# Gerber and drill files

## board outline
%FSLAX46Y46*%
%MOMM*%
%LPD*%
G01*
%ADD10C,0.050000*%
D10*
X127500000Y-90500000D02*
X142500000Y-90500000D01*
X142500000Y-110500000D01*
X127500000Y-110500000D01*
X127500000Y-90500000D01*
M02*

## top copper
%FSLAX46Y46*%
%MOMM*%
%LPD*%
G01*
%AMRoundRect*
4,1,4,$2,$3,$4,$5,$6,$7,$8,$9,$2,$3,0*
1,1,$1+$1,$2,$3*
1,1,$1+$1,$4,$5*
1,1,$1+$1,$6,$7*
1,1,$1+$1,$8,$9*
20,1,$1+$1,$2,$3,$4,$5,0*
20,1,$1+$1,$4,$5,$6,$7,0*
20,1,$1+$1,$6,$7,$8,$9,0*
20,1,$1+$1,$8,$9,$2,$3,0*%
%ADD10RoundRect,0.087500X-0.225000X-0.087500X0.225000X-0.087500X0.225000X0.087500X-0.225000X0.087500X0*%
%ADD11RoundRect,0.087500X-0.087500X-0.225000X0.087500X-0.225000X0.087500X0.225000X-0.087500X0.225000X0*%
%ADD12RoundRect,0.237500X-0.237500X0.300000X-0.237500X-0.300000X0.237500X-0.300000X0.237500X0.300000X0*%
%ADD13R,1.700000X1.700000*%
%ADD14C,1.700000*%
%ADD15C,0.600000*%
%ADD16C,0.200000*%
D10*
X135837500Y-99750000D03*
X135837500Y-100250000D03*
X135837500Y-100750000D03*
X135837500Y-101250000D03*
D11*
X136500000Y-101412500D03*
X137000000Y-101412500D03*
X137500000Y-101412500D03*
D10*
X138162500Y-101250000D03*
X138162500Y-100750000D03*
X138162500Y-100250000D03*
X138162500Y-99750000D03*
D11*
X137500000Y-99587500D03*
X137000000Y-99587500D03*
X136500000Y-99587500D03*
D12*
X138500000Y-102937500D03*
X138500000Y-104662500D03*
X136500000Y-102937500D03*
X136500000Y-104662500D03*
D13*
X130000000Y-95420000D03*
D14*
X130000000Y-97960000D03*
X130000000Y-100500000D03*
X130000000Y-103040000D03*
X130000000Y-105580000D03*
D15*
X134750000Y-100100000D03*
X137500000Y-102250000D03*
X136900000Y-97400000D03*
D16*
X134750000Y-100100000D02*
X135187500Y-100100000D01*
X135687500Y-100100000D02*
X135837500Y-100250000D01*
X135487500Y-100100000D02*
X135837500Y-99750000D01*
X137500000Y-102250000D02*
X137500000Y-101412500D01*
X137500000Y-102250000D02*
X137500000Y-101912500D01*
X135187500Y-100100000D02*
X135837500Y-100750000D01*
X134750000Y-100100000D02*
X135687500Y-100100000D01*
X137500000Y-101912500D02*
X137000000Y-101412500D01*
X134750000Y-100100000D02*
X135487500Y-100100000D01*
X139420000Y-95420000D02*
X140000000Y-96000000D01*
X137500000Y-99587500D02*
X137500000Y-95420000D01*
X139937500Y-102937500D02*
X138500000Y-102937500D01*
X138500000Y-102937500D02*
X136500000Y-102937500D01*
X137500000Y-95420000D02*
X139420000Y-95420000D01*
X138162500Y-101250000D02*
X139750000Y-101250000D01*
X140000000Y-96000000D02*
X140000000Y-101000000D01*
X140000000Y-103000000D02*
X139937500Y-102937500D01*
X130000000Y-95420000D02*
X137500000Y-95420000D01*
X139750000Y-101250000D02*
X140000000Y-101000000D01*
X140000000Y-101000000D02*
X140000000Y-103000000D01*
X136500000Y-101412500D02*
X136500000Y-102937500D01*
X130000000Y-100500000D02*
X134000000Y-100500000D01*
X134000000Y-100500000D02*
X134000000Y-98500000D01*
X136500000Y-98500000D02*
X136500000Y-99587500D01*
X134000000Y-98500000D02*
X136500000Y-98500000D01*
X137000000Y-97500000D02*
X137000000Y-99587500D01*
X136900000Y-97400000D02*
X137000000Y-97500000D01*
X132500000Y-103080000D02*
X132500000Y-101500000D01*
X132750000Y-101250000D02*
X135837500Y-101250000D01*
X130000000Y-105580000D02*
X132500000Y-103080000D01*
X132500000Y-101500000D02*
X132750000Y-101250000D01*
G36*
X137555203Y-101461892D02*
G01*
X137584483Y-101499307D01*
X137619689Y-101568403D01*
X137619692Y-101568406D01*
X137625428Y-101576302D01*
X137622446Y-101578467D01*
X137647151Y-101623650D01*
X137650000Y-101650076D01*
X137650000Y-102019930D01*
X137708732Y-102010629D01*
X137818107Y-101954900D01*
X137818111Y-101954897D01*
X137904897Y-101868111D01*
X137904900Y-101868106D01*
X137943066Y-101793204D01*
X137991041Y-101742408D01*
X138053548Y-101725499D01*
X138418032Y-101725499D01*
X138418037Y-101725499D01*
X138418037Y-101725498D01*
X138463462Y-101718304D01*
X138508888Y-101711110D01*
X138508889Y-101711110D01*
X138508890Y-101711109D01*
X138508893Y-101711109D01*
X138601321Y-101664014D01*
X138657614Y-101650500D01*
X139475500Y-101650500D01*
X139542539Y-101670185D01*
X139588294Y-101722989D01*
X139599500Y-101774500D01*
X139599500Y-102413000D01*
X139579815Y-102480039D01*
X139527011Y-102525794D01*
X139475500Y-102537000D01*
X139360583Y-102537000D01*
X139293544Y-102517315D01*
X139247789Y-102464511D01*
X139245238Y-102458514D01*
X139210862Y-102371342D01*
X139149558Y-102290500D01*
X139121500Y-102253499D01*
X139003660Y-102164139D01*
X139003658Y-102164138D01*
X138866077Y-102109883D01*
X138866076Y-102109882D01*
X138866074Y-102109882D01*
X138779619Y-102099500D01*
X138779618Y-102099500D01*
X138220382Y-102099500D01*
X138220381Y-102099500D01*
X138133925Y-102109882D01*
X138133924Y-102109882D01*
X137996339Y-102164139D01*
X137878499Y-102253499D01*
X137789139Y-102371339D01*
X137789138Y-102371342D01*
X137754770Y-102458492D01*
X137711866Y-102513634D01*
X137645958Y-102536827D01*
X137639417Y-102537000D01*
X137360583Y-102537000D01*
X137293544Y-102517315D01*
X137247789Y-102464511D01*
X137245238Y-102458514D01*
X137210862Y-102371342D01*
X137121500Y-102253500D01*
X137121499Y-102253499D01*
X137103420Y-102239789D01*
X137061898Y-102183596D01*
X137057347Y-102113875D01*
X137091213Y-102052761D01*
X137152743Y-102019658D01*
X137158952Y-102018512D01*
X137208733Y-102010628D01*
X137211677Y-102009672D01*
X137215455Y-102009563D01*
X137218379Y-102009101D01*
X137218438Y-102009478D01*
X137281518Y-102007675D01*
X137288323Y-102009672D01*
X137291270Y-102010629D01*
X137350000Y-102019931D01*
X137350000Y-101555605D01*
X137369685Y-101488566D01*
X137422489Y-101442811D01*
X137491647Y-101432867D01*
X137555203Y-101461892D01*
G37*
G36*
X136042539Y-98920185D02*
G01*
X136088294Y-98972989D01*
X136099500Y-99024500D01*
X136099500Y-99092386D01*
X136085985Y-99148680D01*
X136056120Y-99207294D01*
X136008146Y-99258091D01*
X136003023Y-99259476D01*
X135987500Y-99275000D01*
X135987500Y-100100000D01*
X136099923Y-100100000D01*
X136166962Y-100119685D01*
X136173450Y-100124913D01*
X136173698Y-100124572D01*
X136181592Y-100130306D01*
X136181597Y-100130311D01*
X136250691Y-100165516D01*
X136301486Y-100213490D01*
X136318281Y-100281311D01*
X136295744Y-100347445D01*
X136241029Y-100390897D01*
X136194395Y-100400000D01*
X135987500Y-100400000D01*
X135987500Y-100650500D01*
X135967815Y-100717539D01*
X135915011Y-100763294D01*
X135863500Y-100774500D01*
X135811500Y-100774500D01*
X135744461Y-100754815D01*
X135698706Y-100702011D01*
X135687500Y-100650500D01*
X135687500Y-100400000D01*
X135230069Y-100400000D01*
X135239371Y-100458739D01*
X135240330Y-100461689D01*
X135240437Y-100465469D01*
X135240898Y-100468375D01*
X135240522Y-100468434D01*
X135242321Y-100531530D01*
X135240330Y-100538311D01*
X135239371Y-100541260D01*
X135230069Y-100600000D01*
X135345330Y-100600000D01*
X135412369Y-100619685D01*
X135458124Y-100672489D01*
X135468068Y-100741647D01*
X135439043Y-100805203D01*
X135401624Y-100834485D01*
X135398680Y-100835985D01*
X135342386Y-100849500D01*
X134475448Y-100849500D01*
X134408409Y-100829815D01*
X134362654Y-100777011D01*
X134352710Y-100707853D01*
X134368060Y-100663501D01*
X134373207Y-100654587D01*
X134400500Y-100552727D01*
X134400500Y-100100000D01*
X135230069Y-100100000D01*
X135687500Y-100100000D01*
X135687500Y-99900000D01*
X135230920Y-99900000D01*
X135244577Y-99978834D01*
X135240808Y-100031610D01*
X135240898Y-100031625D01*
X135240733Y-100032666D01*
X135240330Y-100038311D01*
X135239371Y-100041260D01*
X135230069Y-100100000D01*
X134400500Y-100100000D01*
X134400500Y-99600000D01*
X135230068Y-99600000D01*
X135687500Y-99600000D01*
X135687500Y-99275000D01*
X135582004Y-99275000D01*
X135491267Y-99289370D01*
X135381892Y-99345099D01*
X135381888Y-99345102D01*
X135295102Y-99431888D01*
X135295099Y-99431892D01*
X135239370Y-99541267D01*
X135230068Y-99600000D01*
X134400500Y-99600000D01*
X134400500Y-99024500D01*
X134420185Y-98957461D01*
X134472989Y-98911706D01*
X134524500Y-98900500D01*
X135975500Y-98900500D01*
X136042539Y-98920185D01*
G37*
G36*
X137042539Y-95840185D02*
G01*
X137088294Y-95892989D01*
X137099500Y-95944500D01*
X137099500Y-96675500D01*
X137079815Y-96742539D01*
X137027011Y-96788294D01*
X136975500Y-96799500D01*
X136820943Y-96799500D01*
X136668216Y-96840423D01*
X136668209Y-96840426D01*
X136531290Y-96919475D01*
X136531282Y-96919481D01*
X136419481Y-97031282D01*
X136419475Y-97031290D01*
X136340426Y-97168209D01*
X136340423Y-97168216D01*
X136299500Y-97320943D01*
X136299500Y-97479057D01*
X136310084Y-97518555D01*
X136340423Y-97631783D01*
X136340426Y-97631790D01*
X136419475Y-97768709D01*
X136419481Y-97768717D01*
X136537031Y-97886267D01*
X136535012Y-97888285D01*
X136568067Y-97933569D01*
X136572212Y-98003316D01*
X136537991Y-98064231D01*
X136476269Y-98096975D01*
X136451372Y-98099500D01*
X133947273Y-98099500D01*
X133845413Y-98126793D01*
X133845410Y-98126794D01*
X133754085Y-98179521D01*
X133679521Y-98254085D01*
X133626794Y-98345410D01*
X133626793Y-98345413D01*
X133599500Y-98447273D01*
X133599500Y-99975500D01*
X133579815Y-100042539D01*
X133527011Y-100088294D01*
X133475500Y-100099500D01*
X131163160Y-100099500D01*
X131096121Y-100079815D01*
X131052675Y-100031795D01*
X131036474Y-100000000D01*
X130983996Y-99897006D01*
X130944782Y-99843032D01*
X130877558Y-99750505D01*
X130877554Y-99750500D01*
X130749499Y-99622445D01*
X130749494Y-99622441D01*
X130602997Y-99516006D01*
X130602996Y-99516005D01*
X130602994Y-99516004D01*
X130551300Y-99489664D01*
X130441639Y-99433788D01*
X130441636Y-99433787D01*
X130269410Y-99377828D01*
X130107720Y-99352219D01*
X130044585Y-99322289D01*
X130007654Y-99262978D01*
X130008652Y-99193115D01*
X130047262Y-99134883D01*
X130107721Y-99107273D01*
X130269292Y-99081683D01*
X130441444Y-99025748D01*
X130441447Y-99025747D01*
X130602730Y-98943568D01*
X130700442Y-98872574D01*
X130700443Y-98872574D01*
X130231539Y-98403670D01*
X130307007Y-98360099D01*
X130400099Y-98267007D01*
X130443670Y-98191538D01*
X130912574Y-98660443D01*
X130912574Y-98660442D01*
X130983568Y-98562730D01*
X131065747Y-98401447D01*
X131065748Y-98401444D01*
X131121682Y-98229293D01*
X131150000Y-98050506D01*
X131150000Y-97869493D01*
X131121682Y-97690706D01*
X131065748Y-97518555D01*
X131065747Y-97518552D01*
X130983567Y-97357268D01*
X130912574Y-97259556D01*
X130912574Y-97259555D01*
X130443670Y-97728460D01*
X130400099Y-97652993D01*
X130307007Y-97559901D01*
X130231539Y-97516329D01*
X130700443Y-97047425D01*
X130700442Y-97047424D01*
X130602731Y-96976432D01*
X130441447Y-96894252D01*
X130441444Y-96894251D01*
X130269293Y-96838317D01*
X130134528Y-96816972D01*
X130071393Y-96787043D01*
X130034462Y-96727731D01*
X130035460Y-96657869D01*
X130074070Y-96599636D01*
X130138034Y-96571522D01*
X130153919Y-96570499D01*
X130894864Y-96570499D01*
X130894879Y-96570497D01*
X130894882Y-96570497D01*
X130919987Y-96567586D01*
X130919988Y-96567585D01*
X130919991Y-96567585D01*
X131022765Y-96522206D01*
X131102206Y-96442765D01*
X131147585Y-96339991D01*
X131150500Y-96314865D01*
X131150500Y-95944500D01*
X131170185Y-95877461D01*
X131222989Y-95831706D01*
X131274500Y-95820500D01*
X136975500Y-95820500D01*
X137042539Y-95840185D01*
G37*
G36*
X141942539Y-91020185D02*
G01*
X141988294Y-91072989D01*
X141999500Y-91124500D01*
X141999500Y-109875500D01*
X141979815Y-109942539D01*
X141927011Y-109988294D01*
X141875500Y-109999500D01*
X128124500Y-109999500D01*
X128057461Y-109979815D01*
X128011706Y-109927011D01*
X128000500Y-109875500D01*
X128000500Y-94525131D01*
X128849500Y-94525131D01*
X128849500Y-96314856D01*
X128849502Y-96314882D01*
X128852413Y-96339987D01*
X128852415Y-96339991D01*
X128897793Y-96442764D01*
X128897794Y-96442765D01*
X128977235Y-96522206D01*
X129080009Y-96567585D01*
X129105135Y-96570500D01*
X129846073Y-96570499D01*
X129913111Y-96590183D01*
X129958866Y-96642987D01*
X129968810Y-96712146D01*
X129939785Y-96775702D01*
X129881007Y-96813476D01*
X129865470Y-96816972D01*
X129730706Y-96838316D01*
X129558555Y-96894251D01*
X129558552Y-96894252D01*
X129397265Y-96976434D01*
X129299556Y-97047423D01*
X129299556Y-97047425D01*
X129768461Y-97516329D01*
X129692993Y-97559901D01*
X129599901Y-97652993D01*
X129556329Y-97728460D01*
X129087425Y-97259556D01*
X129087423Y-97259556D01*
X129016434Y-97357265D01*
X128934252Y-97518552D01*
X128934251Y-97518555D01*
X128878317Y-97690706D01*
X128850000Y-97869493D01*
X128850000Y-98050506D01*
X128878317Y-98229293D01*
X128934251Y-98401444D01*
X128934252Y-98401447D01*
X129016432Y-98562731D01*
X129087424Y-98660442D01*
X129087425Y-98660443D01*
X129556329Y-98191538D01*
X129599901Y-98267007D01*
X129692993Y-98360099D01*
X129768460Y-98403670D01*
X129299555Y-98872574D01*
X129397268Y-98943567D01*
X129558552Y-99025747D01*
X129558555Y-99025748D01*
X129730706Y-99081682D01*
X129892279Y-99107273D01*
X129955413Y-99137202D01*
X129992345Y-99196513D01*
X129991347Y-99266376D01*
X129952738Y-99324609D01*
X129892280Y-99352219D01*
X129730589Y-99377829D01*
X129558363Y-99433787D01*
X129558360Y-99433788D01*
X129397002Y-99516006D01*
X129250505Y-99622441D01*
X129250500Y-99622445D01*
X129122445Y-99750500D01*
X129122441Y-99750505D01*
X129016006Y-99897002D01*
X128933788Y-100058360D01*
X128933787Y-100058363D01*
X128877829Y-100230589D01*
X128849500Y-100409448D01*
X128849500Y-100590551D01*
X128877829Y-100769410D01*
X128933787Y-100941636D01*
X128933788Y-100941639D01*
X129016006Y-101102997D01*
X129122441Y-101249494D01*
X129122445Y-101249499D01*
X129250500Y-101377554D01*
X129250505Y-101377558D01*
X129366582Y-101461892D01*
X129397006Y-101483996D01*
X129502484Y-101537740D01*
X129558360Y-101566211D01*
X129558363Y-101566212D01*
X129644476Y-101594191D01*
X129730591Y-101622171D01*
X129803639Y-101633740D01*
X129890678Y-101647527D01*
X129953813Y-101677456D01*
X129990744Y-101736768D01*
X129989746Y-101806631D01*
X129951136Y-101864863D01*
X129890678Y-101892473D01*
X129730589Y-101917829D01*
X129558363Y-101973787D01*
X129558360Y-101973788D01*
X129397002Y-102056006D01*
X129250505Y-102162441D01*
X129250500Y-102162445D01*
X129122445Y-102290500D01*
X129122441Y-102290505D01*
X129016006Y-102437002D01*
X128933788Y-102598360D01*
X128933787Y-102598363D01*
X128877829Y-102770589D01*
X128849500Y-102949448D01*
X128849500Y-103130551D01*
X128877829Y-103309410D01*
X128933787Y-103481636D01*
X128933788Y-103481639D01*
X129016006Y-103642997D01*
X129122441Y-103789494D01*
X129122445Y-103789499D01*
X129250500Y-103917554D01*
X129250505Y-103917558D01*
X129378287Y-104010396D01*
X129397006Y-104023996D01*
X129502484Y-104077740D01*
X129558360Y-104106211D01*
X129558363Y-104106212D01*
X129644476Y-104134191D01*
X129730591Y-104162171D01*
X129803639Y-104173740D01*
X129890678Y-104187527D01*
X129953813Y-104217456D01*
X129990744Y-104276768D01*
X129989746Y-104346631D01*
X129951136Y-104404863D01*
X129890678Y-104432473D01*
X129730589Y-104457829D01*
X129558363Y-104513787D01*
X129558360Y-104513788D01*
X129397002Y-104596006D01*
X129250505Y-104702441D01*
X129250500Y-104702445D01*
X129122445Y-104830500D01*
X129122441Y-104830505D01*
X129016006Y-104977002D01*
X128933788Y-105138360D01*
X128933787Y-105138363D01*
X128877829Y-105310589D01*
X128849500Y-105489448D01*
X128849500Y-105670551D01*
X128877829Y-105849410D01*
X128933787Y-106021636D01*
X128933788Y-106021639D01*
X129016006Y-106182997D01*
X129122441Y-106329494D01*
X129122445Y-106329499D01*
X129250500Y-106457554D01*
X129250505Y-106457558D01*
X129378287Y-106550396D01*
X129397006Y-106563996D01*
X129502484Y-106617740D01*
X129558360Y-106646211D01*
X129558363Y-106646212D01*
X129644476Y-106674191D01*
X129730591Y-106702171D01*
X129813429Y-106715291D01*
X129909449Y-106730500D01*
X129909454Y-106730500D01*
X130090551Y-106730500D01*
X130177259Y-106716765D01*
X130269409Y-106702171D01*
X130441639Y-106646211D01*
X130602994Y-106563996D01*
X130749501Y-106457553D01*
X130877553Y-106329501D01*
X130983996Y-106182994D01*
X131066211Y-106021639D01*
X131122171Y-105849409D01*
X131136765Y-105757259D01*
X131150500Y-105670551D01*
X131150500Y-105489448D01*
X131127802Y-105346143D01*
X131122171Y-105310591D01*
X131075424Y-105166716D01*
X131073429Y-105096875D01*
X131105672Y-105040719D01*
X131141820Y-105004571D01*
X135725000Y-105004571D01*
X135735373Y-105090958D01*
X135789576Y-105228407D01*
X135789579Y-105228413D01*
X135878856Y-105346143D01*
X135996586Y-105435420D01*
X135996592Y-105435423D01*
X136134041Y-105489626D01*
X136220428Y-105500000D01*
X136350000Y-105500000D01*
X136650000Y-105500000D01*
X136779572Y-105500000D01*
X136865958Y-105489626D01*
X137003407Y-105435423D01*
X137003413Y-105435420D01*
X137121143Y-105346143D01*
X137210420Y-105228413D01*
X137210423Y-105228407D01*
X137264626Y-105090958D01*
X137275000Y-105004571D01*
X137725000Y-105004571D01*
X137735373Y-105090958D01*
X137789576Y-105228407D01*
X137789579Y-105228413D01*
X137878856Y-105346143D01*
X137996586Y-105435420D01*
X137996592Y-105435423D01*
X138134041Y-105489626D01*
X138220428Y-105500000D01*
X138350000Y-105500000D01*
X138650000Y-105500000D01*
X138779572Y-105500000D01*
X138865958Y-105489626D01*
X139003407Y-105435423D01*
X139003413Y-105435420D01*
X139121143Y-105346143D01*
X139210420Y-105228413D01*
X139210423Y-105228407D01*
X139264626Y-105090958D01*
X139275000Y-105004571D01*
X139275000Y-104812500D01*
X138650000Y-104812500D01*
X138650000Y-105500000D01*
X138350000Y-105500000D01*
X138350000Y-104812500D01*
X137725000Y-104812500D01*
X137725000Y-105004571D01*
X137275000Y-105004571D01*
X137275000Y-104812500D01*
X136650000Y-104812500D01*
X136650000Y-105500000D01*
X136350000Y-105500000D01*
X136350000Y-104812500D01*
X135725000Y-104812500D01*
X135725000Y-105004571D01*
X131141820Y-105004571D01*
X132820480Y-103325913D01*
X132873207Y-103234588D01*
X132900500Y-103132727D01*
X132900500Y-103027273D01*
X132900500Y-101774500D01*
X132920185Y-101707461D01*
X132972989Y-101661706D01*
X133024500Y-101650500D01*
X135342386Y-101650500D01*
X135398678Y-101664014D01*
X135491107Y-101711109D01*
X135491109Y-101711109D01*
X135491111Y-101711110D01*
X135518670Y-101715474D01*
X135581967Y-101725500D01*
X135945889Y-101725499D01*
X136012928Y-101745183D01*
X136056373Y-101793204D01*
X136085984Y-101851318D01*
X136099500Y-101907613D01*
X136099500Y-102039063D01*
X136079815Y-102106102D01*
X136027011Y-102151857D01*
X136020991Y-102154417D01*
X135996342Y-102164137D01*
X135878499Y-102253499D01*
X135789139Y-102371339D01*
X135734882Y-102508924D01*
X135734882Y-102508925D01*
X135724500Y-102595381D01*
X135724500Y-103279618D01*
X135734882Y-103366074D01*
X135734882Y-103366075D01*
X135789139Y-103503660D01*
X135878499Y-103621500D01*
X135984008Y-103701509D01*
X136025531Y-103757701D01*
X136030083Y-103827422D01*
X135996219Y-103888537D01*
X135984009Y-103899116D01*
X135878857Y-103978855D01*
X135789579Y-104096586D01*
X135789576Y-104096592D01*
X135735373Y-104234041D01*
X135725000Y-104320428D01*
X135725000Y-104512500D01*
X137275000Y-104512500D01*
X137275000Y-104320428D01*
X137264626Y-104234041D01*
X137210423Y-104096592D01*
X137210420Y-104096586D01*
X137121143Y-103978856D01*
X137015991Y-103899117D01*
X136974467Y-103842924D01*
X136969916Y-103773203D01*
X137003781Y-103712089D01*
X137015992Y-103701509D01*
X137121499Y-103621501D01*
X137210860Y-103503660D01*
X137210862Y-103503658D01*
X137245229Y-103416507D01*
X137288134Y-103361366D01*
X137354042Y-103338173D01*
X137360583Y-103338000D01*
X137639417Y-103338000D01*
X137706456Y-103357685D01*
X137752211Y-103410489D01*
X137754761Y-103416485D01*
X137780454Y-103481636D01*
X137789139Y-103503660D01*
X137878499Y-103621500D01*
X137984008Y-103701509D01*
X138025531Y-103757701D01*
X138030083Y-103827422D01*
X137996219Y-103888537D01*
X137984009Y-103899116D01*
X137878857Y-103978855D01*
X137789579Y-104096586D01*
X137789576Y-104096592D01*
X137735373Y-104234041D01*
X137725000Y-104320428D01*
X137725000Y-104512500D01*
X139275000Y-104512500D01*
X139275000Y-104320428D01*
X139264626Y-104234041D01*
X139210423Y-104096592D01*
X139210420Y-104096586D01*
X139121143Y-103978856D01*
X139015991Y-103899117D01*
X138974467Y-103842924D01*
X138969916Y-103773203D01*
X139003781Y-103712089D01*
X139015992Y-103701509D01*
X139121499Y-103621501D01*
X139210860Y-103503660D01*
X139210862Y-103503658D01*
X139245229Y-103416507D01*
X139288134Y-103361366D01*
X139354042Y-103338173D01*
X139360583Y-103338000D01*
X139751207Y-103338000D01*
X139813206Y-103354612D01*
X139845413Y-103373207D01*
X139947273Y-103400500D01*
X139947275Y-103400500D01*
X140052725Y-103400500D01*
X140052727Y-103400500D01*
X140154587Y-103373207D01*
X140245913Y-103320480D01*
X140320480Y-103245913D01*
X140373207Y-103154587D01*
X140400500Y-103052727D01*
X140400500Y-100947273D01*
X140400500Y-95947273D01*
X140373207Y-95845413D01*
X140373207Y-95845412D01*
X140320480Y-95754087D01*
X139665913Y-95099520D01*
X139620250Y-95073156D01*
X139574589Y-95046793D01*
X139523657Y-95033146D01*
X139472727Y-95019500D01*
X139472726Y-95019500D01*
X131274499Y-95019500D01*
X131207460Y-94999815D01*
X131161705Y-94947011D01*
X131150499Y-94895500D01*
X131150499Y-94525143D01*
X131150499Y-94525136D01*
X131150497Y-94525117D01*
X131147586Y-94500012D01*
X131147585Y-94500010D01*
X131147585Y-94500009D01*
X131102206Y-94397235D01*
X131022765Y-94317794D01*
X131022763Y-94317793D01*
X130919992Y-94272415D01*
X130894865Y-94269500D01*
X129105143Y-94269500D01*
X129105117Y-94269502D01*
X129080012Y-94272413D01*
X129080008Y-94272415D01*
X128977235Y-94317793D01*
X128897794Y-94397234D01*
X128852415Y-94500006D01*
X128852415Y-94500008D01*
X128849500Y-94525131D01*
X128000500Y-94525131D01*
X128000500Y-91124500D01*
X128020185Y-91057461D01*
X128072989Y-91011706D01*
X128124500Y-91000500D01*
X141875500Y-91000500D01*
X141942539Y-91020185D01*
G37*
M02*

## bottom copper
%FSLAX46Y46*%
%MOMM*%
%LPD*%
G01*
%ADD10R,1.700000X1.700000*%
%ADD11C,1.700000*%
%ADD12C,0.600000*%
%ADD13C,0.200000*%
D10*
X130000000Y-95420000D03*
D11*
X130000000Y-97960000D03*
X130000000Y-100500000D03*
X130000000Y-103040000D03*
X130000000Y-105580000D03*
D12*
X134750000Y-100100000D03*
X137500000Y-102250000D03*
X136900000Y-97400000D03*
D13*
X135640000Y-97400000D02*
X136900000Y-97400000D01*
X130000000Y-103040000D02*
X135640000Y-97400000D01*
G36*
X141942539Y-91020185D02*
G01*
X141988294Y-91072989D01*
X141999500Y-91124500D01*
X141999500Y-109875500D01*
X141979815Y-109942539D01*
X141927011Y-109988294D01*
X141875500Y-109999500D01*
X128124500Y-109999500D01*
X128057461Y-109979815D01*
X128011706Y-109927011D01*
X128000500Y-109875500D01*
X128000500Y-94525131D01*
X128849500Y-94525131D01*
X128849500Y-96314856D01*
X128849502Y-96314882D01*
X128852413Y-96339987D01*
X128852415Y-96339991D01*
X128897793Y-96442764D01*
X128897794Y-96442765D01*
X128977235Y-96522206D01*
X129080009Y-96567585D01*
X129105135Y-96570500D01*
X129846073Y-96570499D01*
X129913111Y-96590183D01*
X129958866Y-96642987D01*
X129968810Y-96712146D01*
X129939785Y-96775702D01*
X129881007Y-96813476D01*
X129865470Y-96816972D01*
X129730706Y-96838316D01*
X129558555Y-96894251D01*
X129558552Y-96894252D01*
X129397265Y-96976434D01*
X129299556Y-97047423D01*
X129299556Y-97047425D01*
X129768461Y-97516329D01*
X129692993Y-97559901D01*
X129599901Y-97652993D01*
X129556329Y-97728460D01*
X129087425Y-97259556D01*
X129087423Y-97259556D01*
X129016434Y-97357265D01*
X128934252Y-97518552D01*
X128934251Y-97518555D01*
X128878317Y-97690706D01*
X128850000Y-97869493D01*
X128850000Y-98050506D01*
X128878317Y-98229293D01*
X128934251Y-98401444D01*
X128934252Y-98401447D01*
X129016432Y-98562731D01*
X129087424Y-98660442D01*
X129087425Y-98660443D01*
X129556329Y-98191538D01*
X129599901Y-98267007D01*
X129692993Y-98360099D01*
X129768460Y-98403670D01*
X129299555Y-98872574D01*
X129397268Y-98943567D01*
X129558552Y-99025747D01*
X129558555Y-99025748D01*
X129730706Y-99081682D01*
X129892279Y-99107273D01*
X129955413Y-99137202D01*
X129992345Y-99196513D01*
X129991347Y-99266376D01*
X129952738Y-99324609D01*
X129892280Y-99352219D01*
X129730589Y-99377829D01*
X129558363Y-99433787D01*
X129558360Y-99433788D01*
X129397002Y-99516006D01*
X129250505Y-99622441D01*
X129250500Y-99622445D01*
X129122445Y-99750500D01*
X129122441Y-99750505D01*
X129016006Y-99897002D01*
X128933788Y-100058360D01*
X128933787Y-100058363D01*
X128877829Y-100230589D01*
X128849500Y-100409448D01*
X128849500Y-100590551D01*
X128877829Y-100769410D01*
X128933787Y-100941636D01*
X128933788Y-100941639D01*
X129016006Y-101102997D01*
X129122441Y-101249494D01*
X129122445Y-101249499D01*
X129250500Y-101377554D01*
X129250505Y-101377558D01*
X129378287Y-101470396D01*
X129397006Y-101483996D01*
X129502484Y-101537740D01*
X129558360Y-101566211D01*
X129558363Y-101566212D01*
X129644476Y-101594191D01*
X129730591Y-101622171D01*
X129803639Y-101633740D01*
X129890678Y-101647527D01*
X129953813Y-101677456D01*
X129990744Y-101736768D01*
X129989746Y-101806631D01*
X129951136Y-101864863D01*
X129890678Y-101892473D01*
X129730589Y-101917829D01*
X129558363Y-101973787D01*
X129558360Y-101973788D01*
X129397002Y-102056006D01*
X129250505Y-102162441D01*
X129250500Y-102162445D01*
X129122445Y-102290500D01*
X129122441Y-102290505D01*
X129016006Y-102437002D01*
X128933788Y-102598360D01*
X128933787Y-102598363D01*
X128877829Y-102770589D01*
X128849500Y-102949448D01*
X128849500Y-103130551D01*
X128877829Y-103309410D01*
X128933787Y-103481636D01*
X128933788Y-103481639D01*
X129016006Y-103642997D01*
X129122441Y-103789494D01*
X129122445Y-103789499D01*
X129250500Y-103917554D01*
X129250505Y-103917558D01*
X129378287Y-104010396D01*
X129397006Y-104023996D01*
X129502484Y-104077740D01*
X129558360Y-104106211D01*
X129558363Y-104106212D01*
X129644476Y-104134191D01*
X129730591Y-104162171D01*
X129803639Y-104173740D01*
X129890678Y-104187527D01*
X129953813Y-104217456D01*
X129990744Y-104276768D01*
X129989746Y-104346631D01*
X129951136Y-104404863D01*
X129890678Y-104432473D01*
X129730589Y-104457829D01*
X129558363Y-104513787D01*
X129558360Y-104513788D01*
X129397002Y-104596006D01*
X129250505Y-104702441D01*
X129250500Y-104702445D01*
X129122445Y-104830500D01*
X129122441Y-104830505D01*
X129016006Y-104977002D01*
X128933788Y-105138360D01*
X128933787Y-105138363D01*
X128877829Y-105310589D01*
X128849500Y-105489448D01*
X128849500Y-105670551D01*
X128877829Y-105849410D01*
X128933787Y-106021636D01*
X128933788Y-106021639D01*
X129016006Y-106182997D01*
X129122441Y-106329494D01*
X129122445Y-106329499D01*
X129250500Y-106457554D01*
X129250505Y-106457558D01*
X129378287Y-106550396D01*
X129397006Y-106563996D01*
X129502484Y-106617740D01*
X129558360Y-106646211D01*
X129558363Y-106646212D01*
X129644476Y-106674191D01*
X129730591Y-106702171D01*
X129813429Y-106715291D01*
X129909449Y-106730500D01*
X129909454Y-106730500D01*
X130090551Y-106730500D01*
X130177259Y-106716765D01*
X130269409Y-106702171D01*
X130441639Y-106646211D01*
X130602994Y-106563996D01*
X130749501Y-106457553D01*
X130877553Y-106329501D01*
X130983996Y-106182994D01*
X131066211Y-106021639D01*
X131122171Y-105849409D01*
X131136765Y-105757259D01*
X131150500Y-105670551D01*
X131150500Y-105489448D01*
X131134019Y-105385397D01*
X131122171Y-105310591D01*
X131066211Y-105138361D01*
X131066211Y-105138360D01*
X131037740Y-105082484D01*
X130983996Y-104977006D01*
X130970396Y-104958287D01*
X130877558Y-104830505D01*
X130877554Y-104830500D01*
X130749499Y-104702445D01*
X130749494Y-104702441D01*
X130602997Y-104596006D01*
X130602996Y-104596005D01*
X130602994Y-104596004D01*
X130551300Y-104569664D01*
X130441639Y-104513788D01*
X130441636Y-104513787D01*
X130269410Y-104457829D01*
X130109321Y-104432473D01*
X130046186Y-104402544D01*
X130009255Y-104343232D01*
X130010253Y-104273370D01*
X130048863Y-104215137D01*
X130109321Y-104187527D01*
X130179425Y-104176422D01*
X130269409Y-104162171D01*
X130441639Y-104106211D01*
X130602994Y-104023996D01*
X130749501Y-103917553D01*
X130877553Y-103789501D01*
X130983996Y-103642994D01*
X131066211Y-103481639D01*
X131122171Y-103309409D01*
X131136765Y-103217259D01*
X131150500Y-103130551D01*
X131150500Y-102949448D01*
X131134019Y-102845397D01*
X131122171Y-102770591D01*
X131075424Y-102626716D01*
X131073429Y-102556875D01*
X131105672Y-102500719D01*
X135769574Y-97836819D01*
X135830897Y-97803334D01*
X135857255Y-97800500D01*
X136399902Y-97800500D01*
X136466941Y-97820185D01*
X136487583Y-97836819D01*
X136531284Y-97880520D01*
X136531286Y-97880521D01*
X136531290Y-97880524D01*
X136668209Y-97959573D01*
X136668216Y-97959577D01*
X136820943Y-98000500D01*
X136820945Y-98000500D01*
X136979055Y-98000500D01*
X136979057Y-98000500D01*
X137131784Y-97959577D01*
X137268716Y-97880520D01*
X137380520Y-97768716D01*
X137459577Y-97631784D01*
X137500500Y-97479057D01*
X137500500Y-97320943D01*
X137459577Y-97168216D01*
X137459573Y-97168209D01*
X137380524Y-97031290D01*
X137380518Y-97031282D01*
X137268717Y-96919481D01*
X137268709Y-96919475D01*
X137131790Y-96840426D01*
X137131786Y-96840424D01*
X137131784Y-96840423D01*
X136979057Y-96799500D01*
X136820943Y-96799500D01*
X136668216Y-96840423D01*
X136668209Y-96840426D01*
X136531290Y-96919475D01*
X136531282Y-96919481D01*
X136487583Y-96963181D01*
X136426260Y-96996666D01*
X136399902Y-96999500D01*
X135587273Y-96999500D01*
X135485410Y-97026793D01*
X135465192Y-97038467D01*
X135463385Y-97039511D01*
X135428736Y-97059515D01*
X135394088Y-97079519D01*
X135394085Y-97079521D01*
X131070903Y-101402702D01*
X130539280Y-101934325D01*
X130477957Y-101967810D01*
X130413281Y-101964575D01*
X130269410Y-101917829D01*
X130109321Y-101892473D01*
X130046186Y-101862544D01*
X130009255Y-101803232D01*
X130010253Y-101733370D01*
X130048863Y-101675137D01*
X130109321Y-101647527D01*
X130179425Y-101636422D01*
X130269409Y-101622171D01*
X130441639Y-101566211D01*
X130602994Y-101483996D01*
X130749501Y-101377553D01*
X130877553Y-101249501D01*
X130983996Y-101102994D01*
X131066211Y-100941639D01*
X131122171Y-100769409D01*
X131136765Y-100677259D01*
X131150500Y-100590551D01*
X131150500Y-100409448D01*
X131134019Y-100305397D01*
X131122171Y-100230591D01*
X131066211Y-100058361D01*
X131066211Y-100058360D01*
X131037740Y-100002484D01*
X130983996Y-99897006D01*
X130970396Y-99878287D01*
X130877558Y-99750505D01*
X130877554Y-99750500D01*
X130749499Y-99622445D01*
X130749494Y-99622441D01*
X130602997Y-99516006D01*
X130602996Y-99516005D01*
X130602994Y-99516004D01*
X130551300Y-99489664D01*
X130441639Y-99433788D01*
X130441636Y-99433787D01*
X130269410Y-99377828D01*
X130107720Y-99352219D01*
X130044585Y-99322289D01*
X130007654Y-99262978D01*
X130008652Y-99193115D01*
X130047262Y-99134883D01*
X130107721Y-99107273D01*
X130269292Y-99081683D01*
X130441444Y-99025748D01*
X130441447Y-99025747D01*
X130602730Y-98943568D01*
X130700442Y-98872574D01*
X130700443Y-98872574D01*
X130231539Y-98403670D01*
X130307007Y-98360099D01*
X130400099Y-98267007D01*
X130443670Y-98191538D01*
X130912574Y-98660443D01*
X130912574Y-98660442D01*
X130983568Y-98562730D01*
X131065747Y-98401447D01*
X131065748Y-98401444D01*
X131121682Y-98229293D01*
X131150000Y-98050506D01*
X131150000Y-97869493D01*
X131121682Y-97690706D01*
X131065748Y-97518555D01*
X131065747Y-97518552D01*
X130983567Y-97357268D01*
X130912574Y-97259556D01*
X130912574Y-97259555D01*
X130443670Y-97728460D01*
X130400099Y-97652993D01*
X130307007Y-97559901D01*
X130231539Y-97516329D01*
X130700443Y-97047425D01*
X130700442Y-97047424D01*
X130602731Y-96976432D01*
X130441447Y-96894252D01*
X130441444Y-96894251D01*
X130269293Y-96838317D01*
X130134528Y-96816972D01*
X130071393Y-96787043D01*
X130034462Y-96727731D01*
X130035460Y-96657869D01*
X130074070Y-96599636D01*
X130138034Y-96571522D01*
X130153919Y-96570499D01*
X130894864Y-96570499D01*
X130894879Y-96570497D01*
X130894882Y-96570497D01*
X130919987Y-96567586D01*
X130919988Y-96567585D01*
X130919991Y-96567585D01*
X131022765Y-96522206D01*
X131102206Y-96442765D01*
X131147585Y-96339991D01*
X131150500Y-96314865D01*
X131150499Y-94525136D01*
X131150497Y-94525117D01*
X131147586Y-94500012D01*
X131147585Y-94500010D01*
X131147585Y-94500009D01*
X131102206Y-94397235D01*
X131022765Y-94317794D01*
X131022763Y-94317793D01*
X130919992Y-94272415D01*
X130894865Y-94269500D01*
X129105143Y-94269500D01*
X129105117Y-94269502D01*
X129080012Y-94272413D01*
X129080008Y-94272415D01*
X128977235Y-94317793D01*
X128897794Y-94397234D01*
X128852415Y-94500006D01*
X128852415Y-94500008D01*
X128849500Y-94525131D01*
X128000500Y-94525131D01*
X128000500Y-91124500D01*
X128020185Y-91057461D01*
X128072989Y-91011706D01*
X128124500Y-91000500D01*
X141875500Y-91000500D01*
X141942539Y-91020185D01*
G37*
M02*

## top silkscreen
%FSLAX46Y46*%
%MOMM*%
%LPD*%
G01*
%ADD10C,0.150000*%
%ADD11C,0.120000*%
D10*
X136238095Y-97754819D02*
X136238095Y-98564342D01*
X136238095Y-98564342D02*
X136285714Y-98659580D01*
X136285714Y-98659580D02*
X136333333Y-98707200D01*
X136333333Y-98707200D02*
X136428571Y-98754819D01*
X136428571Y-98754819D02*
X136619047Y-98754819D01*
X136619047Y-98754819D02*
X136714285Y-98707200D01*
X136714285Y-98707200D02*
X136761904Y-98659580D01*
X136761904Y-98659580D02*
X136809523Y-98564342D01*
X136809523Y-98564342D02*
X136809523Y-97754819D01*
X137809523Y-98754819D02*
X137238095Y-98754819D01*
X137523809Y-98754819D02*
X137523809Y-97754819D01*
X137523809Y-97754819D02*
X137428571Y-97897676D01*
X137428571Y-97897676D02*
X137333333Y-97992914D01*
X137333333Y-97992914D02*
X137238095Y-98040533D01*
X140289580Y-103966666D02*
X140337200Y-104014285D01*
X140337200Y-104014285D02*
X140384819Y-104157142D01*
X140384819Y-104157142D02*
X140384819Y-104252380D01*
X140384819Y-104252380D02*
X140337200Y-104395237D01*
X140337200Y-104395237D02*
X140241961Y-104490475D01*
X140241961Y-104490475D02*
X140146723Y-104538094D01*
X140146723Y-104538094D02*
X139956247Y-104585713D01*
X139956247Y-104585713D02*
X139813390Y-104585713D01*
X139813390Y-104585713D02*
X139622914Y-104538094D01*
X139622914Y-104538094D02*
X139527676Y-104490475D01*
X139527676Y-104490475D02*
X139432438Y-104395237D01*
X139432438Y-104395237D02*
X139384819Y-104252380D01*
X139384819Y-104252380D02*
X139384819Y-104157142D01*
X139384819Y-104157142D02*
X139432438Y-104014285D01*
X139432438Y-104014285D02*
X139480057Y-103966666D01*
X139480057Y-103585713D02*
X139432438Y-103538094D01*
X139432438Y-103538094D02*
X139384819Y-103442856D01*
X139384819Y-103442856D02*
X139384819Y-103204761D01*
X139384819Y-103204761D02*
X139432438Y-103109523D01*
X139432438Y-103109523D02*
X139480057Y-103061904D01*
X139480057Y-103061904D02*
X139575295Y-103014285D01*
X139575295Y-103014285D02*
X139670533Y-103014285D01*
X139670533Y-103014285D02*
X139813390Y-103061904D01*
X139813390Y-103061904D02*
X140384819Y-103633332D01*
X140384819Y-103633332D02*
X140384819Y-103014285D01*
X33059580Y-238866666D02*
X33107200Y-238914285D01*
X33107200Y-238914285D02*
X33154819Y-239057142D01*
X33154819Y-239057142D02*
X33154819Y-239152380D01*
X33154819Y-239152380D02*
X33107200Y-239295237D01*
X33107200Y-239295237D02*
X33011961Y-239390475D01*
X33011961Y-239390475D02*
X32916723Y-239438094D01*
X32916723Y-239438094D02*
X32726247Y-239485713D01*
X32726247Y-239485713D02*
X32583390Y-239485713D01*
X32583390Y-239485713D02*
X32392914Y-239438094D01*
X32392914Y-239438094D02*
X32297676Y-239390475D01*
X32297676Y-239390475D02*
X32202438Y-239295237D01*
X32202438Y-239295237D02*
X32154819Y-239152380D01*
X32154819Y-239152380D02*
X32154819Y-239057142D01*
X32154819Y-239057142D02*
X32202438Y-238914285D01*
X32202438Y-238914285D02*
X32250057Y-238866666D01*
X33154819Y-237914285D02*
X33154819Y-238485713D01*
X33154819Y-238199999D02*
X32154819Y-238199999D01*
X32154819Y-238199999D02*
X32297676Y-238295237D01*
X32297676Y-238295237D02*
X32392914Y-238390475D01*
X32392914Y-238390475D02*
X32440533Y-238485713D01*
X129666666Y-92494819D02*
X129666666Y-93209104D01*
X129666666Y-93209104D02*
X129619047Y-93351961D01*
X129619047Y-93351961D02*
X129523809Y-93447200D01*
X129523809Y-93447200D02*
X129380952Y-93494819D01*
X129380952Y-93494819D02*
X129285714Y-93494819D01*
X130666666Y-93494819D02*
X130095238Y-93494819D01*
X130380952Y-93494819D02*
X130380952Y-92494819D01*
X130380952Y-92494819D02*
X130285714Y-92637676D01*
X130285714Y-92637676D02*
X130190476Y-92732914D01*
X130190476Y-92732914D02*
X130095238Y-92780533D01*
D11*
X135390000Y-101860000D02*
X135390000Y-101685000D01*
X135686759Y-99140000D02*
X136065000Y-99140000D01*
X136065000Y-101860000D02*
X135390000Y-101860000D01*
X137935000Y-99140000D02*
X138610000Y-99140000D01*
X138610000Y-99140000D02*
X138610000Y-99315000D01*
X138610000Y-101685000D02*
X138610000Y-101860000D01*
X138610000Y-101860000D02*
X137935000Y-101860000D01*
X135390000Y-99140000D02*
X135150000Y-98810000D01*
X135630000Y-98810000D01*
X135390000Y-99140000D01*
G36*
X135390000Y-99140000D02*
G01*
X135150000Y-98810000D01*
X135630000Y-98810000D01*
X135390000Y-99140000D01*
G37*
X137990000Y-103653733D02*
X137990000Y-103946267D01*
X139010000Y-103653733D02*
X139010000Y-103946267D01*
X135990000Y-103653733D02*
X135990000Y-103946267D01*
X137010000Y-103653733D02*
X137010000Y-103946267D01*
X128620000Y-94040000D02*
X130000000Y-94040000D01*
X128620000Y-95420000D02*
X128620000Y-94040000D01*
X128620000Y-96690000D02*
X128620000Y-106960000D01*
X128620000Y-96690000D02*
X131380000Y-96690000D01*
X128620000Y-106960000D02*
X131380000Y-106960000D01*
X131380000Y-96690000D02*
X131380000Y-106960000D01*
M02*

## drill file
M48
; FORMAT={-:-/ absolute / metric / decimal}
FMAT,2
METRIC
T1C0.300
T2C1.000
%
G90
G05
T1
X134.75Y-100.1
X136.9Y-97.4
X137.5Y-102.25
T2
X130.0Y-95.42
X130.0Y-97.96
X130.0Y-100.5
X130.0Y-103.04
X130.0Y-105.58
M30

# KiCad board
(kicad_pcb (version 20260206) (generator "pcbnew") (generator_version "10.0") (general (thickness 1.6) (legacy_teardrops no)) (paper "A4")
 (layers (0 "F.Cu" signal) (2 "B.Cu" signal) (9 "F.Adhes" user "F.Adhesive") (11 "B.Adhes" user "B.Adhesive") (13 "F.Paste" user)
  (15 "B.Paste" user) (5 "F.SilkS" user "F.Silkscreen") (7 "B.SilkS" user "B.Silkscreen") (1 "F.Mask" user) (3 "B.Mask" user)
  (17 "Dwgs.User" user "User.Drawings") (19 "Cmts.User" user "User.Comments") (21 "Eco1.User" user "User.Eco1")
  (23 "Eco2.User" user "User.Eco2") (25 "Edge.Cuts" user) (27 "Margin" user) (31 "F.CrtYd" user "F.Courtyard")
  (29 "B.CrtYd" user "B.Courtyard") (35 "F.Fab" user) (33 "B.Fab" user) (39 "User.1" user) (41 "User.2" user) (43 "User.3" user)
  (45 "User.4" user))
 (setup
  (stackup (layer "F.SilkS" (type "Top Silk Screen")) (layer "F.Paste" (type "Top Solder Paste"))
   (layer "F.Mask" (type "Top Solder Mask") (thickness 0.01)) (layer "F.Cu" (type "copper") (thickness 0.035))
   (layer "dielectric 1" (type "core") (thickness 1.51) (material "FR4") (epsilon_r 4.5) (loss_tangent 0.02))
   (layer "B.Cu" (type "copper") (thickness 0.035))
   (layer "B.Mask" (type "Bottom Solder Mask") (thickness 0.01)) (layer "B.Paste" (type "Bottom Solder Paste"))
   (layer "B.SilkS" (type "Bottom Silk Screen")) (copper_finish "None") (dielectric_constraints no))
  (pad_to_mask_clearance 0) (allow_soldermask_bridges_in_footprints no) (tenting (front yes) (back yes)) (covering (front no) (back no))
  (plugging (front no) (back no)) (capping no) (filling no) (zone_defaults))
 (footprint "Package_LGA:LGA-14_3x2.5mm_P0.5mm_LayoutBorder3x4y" (layer "F.Cu") (at 137 100.5)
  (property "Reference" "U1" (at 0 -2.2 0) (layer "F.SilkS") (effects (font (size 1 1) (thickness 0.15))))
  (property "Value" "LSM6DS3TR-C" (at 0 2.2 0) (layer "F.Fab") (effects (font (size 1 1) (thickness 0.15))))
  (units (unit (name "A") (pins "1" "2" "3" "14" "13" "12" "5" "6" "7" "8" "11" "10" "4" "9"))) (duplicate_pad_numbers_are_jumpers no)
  (fp_line (start -1.61 1.36) (end -1.61 1.185) (stroke (width 0.12) (type solid)) (layer "F.SilkS"))
  (fp_line (start -1.313241 -1.36) (end -0.935 -1.36) (stroke (width 0.12) (type solid)) (layer "F.SilkS"))
  (fp_line (start -0.935 1.36) (end -1.61 1.36) (stroke (width 0.12) (type solid)) (layer "F.SilkS"))
  (fp_line (start 0.935 -1.36) (end 1.61 -1.36) (stroke (width 0.12) (type solid)) (layer "F.SilkS"))
  (fp_line (start 1.61 -1.36) (end 1.61 -1.185) (stroke (width 0.12) (type solid)) (layer "F.SilkS"))
  (fp_line (start 1.61 1.185) (end 1.61 1.36) (stroke (width 0.12) (type solid)) (layer "F.SilkS"))
  (fp_line (start 1.61 1.36) (end 0.935 1.36) (stroke (width 0.12) (type solid)) (layer "F.SilkS"))
  (fp_poly (pts (xy -1.61 -1.36) (xy -1.85 -1.69) (xy -1.37 -1.69)) (stroke (width 0.12) (type solid)) (fill yes) (layer "F.SilkS"))
  (pad "1" smd roundrect (at -1.1625 -0.75) (size 0.625 0.35) (layers "F.Cu" "F.Mask" "F.Paste") (roundrect_rratio 0.25) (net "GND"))
  (pad "2" smd roundrect (at -1.1625 -0.25) (size 0.625 0.35) (layers "F.Cu" "F.Mask" "F.Paste") (roundrect_rratio 0.25) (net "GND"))
  (pad "3" smd roundrect (at -1.1625 0.25) (size 0.625 0.35) (layers "F.Cu" "F.Mask" "F.Paste") (roundrect_rratio 0.25) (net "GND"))
  (pad "4" smd roundrect (at -1.1625 0.75) (size 0.625 0.35) (layers "F.Cu" "F.Mask" "F.Paste") (roundrect_rratio 0.25)
   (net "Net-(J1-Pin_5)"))
  (pad "5" smd roundrect (at -0.5 0.9125) (size 0.35 0.625) (layers "F.Cu" "F.Mask" "F.Paste") (roundrect_rratio 0.25) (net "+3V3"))
  (pad "6" smd roundrect (at 0 0.9125) (size 0.35 0.625) (layers "F.Cu" "F.Mask" "F.Paste") (roundrect_rratio 0.25) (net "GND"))
  (pad "7" smd roundrect (at 0.5 0.9125) (size 0.35 0.625) (layers "F.Cu" "F.Mask" "F.Paste") (roundrect_rratio 0.25) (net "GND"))
  (pad "8" smd roundrect (at 1.1625 0.75) (size 0.625 0.35) (layers "F.Cu" "F.Mask" "F.Paste") (roundrect_rratio 0.25) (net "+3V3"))
  (pad "9" smd roundrect (at 1.1625 0.25) (size 0.625 0.35) (layers "F.Cu" "F.Mask" "F.Paste") (roundrect_rratio 0.25)
   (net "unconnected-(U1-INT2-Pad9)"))
  (pad "10" smd roundrect (at 1.1625 -0.25) (size 0.625 0.35) (layers "F.Cu" "F.Mask" "F.Paste") (roundrect_rratio 0.25)
   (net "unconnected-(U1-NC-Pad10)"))
  (pad "11" smd roundrect (at 1.1625 -0.75) (size 0.625 0.35) (layers "F.Cu" "F.Mask" "F.Paste") (roundrect_rratio 0.25)
   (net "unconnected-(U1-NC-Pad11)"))
  (pad "12" smd roundrect (at 0.5 -0.9125) (size 0.35 0.625) (layers "F.Cu" "F.Mask" "F.Paste") (roundrect_rratio 0.25) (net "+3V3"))
  (pad "13" smd roundrect (at 0 -0.9125) (size 0.35 0.625) (layers "F.Cu" "F.Mask" "F.Paste") (roundrect_rratio 0.25) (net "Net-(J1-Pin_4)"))
  (pad "14" smd roundrect (at -0.5 -0.9125) (size 0.35 0.625) (layers "F.Cu" "F.Mask" "F.Paste") (roundrect_rratio 0.25)
   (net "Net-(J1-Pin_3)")))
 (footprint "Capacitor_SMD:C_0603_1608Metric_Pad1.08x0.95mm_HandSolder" (layer "F.Cu") (at 138.5 103.8 -90)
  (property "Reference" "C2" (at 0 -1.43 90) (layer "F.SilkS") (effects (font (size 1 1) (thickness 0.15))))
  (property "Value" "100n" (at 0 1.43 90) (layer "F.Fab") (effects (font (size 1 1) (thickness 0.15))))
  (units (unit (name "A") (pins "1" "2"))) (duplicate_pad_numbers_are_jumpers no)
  (fp_line (start -0.146267 0.51) (end 0.146267 0.51) (stroke (width 0.12) (type solid)) (layer "F.SilkS"))
  (fp_line (start -0.146267 -0.51) (end 0.146267 -0.51) (stroke (width 0.12) (type solid)) (layer "F.SilkS"))
  (pad "1" smd roundrect (at -0.8625 0 270) (size 1.075 0.95) (layers "F.Cu" "F.Mask" "F.Paste") (roundrect_rratio 0.25) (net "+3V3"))
  (pad "2" smd roundrect (at 0.8625 0 270) (size 1.075 0.95) (layers "F.Cu" "F.Mask" "F.Paste") (roundrect_rratio 0.25) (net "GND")))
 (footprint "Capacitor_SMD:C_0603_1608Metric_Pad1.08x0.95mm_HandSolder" (layer "F.Cu") (at 136.5 103.8 -90)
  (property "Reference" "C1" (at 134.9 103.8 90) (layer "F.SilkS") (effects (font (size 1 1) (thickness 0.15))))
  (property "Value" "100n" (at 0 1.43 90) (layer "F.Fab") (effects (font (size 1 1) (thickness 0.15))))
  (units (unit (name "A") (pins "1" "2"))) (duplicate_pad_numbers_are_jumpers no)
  (fp_line (start -0.146267 0.51) (end 0.146267 0.51) (stroke (width 0.12) (type solid)) (layer "F.SilkS"))
  (fp_line (start -0.146267 -0.51) (end 0.146267 -0.51) (stroke (width 0.12) (type solid)) (layer "F.SilkS"))
  (pad "1" smd roundrect (at -0.8625 0 270) (size 1.075 0.95) (layers "F.Cu" "F.Mask" "F.Paste") (roundrect_rratio 0.25) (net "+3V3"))
  (pad "2" smd roundrect (at 0.8625 0 270) (size 1.075 0.95) (layers "F.Cu" "F.Mask" "F.Paste") (roundrect_rratio 0.25) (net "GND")))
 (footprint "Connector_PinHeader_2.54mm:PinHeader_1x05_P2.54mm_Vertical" (layer "F.Cu") (at 130 95.42)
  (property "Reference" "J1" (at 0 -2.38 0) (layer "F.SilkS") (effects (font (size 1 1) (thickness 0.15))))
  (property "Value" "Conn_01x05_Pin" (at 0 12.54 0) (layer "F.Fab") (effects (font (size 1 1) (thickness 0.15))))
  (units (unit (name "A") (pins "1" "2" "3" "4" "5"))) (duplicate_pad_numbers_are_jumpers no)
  (fp_line (start -1.38 -1.38) (end 0 -1.38) (stroke (width 0.12) (type solid)) (layer "F.SilkS"))
  (fp_line (start -1.38 0) (end -1.38 -1.38) (stroke (width 0.12) (type solid)) (layer "F.SilkS"))
  (fp_line (start -1.38 1.27) (end -1.38 11.54) (stroke (width 0.12) (type solid)) (layer "F.SilkS"))
  (fp_line (start -1.38 1.27) (end 1.38 1.27) (stroke (width 0.12) (type solid)) (layer "F.SilkS"))
  (fp_line (start -1.38 11.54) (end 1.38 11.54) (stroke (width 0.12) (type solid)) (layer "F.SilkS"))
  (fp_line (start 1.38 1.27) (end 1.38 11.54) (stroke (width 0.12) (type solid)) (layer "F.SilkS"))
  (pad "1" thru_hole rect (at 0 0) (size 1.7 1.7) (drill 1) (layers "*.Cu" "*.Mask") (remove_unused_layers no) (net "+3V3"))
  (pad "2" thru_hole circle (at 0 2.54) (size 1.7 1.7) (drill 1) (layers "*.Cu" "*.Mask") (remove_unused_layers no) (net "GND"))
  (pad "3" thru_hole circle (at 0 5.08) (size 1.7 1.7) (drill 1) (layers "*.Cu" "*.Mask") (remove_unused_layers no) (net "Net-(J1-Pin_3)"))
  (pad "4" thru_hole circle (at 0 7.62) (size 1.7 1.7) (drill 1) (layers "*.Cu" "*.Mask") (remove_unused_layers no) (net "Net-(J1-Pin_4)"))
  (pad "5" thru_hole circle (at 0 10.16) (size 1.7 1.7) (drill 1) (layers "*.Cu" "*.Mask") (remove_unused_layers no) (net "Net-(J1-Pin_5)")))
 (gr_rect (start 127.5 90.5) (end 142.5 110.5) (stroke (width 0.05) (type solid)) (fill no) (layer "Edge.Cuts"))
 (segment (start 134.75 100.1) (end 135.1875 100.1) (width 0.2) (layer "F.Cu") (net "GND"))
 (segment (start 135.6875 100.1) (end 135.8375 100.25) (width 0.2) (layer "F.Cu") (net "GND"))
 (segment (start 135.4875 100.1) (end 135.8375 99.75) (width 0.2) (layer "F.Cu") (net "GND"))
 (segment (start 137.5 102.25) (end 137.5 101.4125) (width 0.2) (layer "F.Cu") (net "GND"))
 (segment (start 137.5 102.25) (end 137.5 101.9125) (width 0.2) (layer "F.Cu") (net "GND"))
 (segment (start 135.1875 100.1) (end 135.8375 100.75) (width 0.2) (layer "F.Cu") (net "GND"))
 (segment (start 134.75 100.1) (end 135.6875 100.1) (width 0.2) (layer "F.Cu") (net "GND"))
 (segment (start 137.5 101.9125) (end 137 101.4125) (width 0.2) (layer "F.Cu") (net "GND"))
 (segment (start 134.75 100.1) (end 135.4875 100.1) (width 0.2) (layer "F.Cu") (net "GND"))
 (via (at 134.75 100.1) (size 0.6) (drill 0.3) (layers "F.Cu" "B.Cu") (free yes) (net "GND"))
 (via (at 137.5 102.25) (size 0.6) (drill 0.3) (layers "F.Cu" "B.Cu") (free yes) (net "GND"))
 (segment (start 139.42 95.42) (end 140 96) (width 0.2) (layer "F.Cu") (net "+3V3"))
 (segment (start 137.5 99.5875) (end 137.5 95.42) (width 0.2) (layer "F.Cu") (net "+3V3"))
 (segment (start 139.9375 102.9375) (end 138.5 102.9375) (width 0.2) (layer "F.Cu") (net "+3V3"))
 (segment (start 138.5 102.9375) (end 136.5 102.9375) (width 0.2) (layer "F.Cu") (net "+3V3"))
 (segment (start 137.5 95.42) (end 139.42 95.42) (width 0.2) (layer "F.Cu") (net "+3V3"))
 (segment (start 138.1625 101.25) (end 139.75 101.25) (width 0.2) (layer "F.Cu") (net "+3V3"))
 (segment (start 140 96) (end 140 101) (width 0.2) (layer "F.Cu") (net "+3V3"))
 (segment (start 140 103) (end 139.9375 102.9375) (width 0.2) (layer "F.Cu") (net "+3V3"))
 (segment (start 130 95.42) (end 137.5 95.42) (width 0.2) (layer "F.Cu") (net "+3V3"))
 (segment (start 139.75 101.25) (end 140 101) (width 0.2) (layer "F.Cu") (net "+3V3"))
 (segment (start 140 101) (end 140 103) (width 0.2) (layer "F.Cu") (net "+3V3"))
 (segment (start 136.5 101.4125) (end 136.5 102.9375) (width 0.2) (layer "F.Cu") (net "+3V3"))
 (segment (start 130 100.5) (end 134 100.5) (width 0.2) (layer "F.Cu") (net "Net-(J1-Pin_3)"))
 (segment (start 134 100.5) (end 134 98.5) (width 0.2) (layer "F.Cu") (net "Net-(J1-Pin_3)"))
 (segment (start 136.5 98.5) (end 136.5 99.5875) (width 0.2) (layer "F.Cu") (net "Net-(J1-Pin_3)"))
 (segment (start 134 98.5) (end 136.5 98.5) (width 0.2) (layer "F.Cu") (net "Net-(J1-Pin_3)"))
 (segment (start 137 97.5) (end 137 99.5875) (width 0.2) (layer "F.Cu") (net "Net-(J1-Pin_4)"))
 (segment (start 136.9 97.4) (end 137 97.5) (width 0.2) (layer "F.Cu") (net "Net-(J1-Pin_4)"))
 (via (at 136.9 97.4) (size 0.6) (drill 0.3) (layers "F.Cu" "B.Cu") (free yes) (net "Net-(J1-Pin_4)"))
 (segment (start 135.64 97.4) (end 136.9 97.4) (width 0.2) (layer "B.Cu") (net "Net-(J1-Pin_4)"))
 (segment (start 130 103.04) (end 135.64 97.4) (width 0.2) (layer "B.Cu") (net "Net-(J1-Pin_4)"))
 (segment (start 132.5 103.08) (end 132.5 101.5) (width 0.2) (layer "F.Cu") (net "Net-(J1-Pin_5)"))
 (segment (start 132.75 101.25) (end 135.8375 101.25) (width 0.2) (layer "F.Cu") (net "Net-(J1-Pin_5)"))
 (segment (start 130 105.58) (end 132.5 103.08) (width 0.2) (layer "F.Cu") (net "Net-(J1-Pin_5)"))
 (segment (start 132.5 101.5) (end 132.75 101.25) (width 0.2) (layer "F.Cu") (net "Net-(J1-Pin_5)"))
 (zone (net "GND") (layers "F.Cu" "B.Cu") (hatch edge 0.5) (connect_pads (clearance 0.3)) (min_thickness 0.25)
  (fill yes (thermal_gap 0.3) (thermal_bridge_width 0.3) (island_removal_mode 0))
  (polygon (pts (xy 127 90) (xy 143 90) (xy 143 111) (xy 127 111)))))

